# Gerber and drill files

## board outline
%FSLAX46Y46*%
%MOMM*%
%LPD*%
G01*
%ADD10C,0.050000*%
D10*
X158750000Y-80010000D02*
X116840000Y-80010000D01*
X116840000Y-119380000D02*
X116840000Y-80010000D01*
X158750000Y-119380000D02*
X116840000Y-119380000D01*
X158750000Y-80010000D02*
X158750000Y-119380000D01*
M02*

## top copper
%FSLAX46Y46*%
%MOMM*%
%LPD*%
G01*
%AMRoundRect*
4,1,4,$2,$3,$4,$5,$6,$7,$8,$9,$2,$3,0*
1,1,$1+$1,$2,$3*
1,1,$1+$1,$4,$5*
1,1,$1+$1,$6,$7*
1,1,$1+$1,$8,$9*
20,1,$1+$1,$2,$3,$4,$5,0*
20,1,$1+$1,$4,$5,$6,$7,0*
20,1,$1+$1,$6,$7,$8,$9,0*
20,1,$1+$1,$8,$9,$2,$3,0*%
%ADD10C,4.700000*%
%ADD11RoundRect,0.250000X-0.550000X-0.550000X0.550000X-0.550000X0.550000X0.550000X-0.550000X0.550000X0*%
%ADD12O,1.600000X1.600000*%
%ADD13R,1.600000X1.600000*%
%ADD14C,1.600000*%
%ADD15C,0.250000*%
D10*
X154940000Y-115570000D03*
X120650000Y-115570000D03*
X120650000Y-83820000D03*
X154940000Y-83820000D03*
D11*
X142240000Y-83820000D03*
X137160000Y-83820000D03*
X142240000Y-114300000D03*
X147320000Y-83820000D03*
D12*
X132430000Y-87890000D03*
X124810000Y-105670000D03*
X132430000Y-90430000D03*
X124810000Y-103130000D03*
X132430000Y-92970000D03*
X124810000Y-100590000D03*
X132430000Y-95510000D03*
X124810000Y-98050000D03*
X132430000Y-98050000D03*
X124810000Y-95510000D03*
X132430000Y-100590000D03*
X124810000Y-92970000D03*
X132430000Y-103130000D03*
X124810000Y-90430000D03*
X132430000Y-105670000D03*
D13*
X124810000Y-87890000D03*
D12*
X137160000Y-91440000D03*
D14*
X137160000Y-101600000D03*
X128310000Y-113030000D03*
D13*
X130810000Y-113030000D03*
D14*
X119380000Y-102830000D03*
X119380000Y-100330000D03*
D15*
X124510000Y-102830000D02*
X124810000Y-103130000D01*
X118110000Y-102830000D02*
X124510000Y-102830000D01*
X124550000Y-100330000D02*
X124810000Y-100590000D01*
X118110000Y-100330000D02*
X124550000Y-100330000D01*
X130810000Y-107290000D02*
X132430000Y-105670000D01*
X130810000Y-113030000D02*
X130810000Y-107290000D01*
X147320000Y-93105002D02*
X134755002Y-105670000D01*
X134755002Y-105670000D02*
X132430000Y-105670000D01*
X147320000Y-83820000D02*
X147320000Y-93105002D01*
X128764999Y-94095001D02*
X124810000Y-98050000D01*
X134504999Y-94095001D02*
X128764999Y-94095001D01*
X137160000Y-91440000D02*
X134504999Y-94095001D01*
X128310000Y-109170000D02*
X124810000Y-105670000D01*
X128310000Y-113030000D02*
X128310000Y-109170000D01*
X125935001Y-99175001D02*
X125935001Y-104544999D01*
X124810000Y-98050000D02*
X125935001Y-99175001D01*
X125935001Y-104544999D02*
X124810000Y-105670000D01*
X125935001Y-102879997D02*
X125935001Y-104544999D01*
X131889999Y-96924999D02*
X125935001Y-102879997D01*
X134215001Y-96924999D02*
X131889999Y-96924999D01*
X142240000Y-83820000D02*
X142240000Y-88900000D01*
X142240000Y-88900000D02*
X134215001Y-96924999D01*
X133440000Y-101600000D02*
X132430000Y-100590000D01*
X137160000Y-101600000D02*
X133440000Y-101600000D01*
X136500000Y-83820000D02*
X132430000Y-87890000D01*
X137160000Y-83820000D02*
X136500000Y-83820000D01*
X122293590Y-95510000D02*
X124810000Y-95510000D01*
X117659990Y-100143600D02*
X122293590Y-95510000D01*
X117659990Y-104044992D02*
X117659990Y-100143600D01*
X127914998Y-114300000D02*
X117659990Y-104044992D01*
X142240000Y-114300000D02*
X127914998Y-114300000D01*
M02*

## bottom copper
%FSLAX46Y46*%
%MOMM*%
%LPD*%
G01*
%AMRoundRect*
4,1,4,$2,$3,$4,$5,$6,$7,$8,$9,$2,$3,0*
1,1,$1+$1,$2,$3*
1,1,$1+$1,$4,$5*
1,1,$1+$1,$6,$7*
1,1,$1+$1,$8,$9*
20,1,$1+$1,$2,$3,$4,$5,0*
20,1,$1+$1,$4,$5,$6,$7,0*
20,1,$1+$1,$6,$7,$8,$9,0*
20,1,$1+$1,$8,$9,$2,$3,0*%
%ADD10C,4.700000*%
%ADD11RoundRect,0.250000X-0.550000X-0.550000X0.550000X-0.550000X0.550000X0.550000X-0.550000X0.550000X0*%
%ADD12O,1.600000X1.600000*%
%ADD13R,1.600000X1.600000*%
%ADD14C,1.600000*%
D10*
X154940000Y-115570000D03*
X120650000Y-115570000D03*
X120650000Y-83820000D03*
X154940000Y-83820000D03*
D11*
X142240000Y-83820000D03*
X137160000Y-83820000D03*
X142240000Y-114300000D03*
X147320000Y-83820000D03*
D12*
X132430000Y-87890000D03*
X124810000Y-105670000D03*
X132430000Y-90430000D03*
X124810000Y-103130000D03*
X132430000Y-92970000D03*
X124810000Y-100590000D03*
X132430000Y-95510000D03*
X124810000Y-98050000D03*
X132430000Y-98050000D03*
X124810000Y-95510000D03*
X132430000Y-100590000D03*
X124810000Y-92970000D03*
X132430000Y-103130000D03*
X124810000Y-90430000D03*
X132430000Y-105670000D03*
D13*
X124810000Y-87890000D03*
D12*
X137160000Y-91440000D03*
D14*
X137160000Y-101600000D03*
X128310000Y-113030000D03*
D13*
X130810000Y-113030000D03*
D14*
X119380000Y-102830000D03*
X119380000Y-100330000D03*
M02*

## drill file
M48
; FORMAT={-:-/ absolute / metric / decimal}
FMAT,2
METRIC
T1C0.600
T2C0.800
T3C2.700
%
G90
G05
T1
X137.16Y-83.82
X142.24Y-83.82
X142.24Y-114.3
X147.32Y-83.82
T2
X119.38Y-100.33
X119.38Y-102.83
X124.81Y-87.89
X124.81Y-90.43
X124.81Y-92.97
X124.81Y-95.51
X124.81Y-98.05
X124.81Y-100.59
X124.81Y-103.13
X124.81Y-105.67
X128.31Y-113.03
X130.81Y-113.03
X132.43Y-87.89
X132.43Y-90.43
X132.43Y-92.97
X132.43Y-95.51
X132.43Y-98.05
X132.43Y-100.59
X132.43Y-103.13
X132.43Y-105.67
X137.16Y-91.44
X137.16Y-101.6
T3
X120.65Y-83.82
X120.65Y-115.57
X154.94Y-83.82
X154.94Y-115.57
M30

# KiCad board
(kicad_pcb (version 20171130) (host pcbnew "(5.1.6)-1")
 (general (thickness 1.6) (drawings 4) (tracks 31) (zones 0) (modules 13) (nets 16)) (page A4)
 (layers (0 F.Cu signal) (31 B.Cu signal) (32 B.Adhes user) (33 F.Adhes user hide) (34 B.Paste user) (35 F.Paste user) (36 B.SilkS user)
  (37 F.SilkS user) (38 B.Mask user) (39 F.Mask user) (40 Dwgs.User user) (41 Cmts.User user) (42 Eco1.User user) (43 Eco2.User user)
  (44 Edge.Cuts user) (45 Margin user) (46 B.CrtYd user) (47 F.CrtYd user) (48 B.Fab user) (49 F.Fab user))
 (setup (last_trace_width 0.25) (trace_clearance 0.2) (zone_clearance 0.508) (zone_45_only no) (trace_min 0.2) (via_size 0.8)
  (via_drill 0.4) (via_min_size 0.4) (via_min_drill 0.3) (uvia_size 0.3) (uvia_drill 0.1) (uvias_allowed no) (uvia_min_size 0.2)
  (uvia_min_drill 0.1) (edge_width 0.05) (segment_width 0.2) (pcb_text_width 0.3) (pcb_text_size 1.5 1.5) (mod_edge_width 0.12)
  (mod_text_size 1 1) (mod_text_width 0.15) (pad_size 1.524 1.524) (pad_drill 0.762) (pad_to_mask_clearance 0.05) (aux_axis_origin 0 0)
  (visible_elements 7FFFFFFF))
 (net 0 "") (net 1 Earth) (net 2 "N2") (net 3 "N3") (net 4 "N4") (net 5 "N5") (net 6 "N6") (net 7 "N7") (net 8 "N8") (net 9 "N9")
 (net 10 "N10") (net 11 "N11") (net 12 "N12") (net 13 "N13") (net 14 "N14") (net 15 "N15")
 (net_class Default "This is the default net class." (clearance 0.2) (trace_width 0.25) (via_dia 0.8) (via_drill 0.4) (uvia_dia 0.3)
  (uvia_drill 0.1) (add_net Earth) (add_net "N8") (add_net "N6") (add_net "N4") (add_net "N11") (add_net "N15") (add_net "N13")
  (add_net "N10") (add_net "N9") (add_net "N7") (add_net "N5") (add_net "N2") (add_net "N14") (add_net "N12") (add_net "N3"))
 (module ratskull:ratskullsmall (layer F.Cu) (at 148.59 100.33)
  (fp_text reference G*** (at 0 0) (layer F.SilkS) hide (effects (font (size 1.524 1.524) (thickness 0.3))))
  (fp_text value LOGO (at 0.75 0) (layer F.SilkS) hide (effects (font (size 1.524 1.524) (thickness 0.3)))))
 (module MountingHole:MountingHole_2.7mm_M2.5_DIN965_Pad (layer F.Cu) (at 154.94 115.57)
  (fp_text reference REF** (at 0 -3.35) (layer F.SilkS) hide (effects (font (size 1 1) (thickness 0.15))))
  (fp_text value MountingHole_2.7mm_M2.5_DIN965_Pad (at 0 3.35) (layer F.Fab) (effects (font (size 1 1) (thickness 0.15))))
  (pad 1 thru_hole circle (at 0 0) (size 4.7 4.7) (drill 2.7) (layers *.Cu *.Mask)))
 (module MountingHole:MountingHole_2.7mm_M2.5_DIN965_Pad (layer F.Cu) (at 120.65 115.57)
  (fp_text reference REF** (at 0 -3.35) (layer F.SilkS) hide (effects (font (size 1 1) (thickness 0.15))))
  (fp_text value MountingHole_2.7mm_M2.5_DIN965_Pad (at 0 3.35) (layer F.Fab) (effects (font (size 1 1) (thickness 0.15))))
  (pad 1 thru_hole circle (at 0 0) (size 4.7 4.7) (drill 2.7) (layers *.Cu *.Mask)))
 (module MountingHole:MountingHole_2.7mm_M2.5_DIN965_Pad (layer F.Cu) (at 120.65 83.82)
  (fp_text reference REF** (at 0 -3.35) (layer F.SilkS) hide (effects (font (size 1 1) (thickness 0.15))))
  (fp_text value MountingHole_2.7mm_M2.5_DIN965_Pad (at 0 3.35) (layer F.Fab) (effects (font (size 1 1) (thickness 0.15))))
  (pad 1 thru_hole circle (at 0 0) (size 4.7 4.7) (drill 2.7) (layers *.Cu *.Mask)))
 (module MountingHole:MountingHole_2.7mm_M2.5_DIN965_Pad (layer F.Cu) (at 154.94 83.82)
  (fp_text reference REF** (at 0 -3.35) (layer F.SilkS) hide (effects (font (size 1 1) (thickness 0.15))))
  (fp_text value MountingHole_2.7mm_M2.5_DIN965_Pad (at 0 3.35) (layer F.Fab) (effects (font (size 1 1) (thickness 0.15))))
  (pad 1 thru_hole circle (at 0 0) (size 4.7 4.7) (drill 2.7) (layers *.Cu *.Mask)))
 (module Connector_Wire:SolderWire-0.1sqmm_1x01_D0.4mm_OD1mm (layer F.Cu) (at 142.24 83.82)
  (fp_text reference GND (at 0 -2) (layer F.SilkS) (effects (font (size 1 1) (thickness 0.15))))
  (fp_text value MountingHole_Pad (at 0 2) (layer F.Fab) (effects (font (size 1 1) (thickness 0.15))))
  (pad 1 thru_hole roundrect (at 0 0) (size 1.6 1.6) (drill 0.6) (layers *.Cu *.Mask) (roundrect_rratio 0.15625) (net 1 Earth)))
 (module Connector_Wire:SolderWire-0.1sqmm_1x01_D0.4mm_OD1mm (layer F.Cu) (at 137.16 83.82)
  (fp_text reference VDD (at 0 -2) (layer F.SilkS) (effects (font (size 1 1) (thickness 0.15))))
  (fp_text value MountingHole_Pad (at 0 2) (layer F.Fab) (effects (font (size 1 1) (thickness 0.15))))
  (pad 1 thru_hole roundrect (at 0 0) (size 1.6 1.6) (drill 0.6) (layers *.Cu *.Mask) (roundrect_rratio 0.15625) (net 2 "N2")))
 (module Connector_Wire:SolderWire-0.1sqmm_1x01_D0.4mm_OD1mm (layer F.Cu) (at 142.24 114.3)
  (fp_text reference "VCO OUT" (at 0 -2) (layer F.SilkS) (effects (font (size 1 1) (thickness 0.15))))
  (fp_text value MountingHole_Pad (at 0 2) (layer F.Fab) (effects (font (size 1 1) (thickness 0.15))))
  (pad 1 thru_hole roundrect (at 0 0) (size 1.6 1.6) (drill 0.6) (layers *.Cu *.Mask) (roundrect_rratio 0.15625) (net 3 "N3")))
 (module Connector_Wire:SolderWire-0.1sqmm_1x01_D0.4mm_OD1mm (layer F.Cu) (at 147.32 83.82)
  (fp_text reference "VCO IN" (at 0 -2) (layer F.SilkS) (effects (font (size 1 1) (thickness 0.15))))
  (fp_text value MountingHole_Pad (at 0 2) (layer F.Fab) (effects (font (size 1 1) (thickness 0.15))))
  (pad 1 thru_hole roundrect (at 0 0) (size 1.6 1.6) (drill 0.6) (layers *.Cu *.Mask) (roundrect_rratio 0.15625) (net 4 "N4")))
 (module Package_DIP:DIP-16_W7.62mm (layer F.Cu) (at 124.81 87.89)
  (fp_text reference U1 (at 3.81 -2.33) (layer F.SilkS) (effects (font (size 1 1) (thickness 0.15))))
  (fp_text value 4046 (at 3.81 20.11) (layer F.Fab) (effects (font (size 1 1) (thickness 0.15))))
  (pad 16 thru_hole oval (at 7.62 0) (size 1.6 1.6) (drill 0.8) (layers *.Cu *.Mask) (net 2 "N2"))
  (pad 8 thru_hole oval (at 0 17.78) (size 1.6 1.6) (drill 0.8) (layers *.Cu *.Mask) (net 1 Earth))
  (pad 15 thru_hole oval (at 7.62 2.54) (size 1.6 1.6) (drill 0.8) (layers *.Cu *.Mask) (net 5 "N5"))
  (pad 7 thru_hole oval (at 0 15.24) (size 1.6 1.6) (drill 0.8) (layers *.Cu *.Mask) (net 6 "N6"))
  (pad 14 thru_hole oval (at 7.62 5.08) (size 1.6 1.6) (drill 0.8) (layers *.Cu *.Mask) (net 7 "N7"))
  (pad 6 thru_hole oval (at 0 12.7) (size 1.6 1.6) (drill 0.8) (layers *.Cu *.Mask) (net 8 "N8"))
  (pad 13 thru_hole oval (at 7.62 7.62) (size 1.6 1.6) (drill 0.8) (layers *.Cu *.Mask) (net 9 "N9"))
  (pad 5 thru_hole oval (at 0 10.16) (size 1.6 1.6) (drill 0.8) (layers *.Cu *.Mask) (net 1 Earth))
  (pad 12 thru_hole oval (at 7.62 10.16) (size 1.6 1.6) (drill 0.8) (layers *.Cu *.Mask) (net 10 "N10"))
  (pad 4 thru_hole oval (at 0 7.62) (size 1.6 1.6) (drill 0.8) (layers *.Cu *.Mask) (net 3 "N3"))
  (pad 11 thru_hole oval (at 7.62 12.7) (size 1.6 1.6) (drill 0.8) (layers *.Cu *.Mask) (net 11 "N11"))
  (pad 3 thru_hole oval (at 0 5.08) (size 1.6 1.6) (drill 0.8) (layers *.Cu *.Mask) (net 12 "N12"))
  (pad 10 thru_hole oval (at 7.62 15.24) (size 1.6 1.6) (drill 0.8) (layers *.Cu *.Mask) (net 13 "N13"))
  (pad 2 thru_hole oval (at 0 2.54) (size 1.6 1.6) (drill 0.8) (layers *.Cu *.Mask) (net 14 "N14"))
  (pad 9 thru_hole oval (at 7.62 17.78) (size 1.6 1.6) (drill 0.8) (layers *.Cu *.Mask) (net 4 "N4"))
  (pad 1 thru_hole rect (at 0 0) (size 1.6 1.6) (drill 0.8) (layers *.Cu *.Mask) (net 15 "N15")))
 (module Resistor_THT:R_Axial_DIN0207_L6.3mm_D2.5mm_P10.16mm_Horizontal (layer F.Cu) (at 137.16 101.6 90)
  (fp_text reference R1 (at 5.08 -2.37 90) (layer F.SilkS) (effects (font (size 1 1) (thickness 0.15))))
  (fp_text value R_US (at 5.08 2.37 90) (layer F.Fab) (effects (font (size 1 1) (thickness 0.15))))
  (pad 2 thru_hole oval (at 10.16 0 90) (size 1.6 1.6) (drill 0.8) (layers *.Cu *.Mask) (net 1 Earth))
  (pad 1 thru_hole circle (at 0 0 90) (size 1.6 1.6) (drill 0.8) (layers *.Cu *.Mask) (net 11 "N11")))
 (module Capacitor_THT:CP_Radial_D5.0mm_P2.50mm (layer F.Cu) (at 130.81 113.03 180)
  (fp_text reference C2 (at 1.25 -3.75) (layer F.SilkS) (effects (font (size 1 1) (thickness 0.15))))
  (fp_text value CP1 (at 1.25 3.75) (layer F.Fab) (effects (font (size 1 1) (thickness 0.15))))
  (pad 2 thru_hole circle (at 2.5 0 180) (size 1.6 1.6) (drill 0.8) (layers *.Cu *.Mask) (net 1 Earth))
  (pad 1 thru_hole rect (at 0 0 180) (size 1.6 1.6) (drill 0.8) (layers *.Cu *.Mask) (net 4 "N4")))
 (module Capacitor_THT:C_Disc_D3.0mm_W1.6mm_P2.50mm (layer F.Cu) (at 119.38 100.33 270)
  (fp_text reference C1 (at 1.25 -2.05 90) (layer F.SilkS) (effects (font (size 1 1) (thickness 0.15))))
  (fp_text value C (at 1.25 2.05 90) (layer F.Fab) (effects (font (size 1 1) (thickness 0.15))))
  (pad 2 thru_hole circle (at 2.5 0 270) (size 1.6 1.6) (drill 0.8) (layers *.Cu *.Mask) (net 6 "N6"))
  (pad 1 thru_hole circle (at 0 0 270) (size 1.6 1.6) (drill 0.8) (layers *.Cu *.Mask) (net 8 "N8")))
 (gr_line (start 158.75 80.01) (end 116.84 80.01) (layer Edge.Cuts) (width 0.05))
 (gr_line (start 116.84 119.38) (end 116.84 80.01) (layer Edge.Cuts) (width 0.05))
 (gr_line (start 158.75 119.38) (end 116.84 119.38) (layer Edge.Cuts) (width 0.05))
 (gr_line (start 158.75 80.01) (end 158.75 119.38) (layer Edge.Cuts) (width 0.05))
 (segment (start 124.51 102.83) (end 124.81 103.13) (width 0.25) (layer F.Cu) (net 6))
 (segment (start 118.11 102.83) (end 124.51 102.83) (width 0.25) (layer F.Cu) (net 6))
 (segment (start 124.55 100.33) (end 124.81 100.59) (width 0.25) (layer F.Cu) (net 8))
 (segment (start 118.11 100.33) (end 124.55 100.33) (width 0.25) (layer F.Cu) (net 8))
 (segment (start 130.81 107.29) (end 132.43 105.67) (width 0.25) (layer F.Cu) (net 4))
 (segment (start 130.81 113.03) (end 130.81 107.29) (width 0.25) (layer F.Cu) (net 4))
 (segment (start 147.32 93.105002) (end 134.755002 105.67) (width 0.25) (layer F.Cu) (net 4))
 (segment (start 134.755002 105.67) (end 132.43 105.67) (width 0.25) (layer F.Cu) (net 4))
 (segment (start 147.32 83.82) (end 147.32 93.105002) (width 0.25) (layer F.Cu) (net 4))
 (segment (start 128.764999 94.095001) (end 124.81 98.05) (width 0.25) (layer F.Cu) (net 1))
 (segment (start 134.504999 94.095001) (end 128.764999 94.095001) (width 0.25) (layer F.Cu) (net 1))
 (segment (start 137.16 91.44) (end 134.504999 94.095001) (width 0.25) (layer F.Cu) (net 1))
 (segment (start 128.31 109.17) (end 124.81 105.67) (width 0.25) (layer F.Cu) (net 1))
 (segment (start 128.31 113.03) (end 128.31 109.17) (width 0.25) (layer F.Cu) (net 1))
 (segment (start 125.935001 99.175001) (end 125.935001 104.544999) (width 0.25) (layer F.Cu) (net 1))
 (segment (start 124.81 98.05) (end 125.935001 99.175001) (width 0.25) (layer F.Cu) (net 1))
 (segment (start 125.935001 104.544999) (end 124.81 105.67) (width 0.25) (layer F.Cu) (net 1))
 (segment (start 125.935001 102.879997) (end 125.935001 104.544999) (width 0.25) (layer F.Cu) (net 1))
 (segment (start 131.889999 96.924999) (end 125.935001 102.879997) (width 0.25) (layer F.Cu) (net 1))
 (segment (start 134.215001 96.924999) (end 131.889999 96.924999) (width 0.25) (layer F.Cu) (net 1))
 (segment (start 142.24 83.82) (end 142.24 88.9) (width 0.25) (layer F.Cu) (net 1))
 (segment (start 142.24 88.9) (end 134.215001 96.924999) (width 0.25) (layer F.Cu) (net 1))
 (segment (start 133.44 101.6) (end 132.43 100.59) (width 0.25) (layer F.Cu) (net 11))
 (segment (start 137.16 101.6) (end 133.44 101.6) (width 0.25) (layer F.Cu) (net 11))
 (segment (start 136.5 83.82) (end 132.43 87.89) (width 0.25) (layer F.Cu) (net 2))
 (segment (start 137.16 83.82) (end 136.5 83.82) (width 0.25) (layer F.Cu) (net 2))
 (segment (start 122.29359 95.51) (end 124.81 95.51) (width 0.25) (layer F.Cu) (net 3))
 (segment (start 117.65999 100.1436) (end 122.29359 95.51) (width 0.25) (layer F.Cu) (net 3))
 (segment (start 117.65999 104.044992) (end 117.65999 100.1436) (width 0.25) (layer F.Cu) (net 3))
 (segment (start 127.914998 114.3) (end 117.65999 104.044992) (width 0.25) (layer F.Cu) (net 3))
 (segment (start 142.24 114.3) (end 127.914998 114.3) (width 0.25) (layer F.Cu) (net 3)))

